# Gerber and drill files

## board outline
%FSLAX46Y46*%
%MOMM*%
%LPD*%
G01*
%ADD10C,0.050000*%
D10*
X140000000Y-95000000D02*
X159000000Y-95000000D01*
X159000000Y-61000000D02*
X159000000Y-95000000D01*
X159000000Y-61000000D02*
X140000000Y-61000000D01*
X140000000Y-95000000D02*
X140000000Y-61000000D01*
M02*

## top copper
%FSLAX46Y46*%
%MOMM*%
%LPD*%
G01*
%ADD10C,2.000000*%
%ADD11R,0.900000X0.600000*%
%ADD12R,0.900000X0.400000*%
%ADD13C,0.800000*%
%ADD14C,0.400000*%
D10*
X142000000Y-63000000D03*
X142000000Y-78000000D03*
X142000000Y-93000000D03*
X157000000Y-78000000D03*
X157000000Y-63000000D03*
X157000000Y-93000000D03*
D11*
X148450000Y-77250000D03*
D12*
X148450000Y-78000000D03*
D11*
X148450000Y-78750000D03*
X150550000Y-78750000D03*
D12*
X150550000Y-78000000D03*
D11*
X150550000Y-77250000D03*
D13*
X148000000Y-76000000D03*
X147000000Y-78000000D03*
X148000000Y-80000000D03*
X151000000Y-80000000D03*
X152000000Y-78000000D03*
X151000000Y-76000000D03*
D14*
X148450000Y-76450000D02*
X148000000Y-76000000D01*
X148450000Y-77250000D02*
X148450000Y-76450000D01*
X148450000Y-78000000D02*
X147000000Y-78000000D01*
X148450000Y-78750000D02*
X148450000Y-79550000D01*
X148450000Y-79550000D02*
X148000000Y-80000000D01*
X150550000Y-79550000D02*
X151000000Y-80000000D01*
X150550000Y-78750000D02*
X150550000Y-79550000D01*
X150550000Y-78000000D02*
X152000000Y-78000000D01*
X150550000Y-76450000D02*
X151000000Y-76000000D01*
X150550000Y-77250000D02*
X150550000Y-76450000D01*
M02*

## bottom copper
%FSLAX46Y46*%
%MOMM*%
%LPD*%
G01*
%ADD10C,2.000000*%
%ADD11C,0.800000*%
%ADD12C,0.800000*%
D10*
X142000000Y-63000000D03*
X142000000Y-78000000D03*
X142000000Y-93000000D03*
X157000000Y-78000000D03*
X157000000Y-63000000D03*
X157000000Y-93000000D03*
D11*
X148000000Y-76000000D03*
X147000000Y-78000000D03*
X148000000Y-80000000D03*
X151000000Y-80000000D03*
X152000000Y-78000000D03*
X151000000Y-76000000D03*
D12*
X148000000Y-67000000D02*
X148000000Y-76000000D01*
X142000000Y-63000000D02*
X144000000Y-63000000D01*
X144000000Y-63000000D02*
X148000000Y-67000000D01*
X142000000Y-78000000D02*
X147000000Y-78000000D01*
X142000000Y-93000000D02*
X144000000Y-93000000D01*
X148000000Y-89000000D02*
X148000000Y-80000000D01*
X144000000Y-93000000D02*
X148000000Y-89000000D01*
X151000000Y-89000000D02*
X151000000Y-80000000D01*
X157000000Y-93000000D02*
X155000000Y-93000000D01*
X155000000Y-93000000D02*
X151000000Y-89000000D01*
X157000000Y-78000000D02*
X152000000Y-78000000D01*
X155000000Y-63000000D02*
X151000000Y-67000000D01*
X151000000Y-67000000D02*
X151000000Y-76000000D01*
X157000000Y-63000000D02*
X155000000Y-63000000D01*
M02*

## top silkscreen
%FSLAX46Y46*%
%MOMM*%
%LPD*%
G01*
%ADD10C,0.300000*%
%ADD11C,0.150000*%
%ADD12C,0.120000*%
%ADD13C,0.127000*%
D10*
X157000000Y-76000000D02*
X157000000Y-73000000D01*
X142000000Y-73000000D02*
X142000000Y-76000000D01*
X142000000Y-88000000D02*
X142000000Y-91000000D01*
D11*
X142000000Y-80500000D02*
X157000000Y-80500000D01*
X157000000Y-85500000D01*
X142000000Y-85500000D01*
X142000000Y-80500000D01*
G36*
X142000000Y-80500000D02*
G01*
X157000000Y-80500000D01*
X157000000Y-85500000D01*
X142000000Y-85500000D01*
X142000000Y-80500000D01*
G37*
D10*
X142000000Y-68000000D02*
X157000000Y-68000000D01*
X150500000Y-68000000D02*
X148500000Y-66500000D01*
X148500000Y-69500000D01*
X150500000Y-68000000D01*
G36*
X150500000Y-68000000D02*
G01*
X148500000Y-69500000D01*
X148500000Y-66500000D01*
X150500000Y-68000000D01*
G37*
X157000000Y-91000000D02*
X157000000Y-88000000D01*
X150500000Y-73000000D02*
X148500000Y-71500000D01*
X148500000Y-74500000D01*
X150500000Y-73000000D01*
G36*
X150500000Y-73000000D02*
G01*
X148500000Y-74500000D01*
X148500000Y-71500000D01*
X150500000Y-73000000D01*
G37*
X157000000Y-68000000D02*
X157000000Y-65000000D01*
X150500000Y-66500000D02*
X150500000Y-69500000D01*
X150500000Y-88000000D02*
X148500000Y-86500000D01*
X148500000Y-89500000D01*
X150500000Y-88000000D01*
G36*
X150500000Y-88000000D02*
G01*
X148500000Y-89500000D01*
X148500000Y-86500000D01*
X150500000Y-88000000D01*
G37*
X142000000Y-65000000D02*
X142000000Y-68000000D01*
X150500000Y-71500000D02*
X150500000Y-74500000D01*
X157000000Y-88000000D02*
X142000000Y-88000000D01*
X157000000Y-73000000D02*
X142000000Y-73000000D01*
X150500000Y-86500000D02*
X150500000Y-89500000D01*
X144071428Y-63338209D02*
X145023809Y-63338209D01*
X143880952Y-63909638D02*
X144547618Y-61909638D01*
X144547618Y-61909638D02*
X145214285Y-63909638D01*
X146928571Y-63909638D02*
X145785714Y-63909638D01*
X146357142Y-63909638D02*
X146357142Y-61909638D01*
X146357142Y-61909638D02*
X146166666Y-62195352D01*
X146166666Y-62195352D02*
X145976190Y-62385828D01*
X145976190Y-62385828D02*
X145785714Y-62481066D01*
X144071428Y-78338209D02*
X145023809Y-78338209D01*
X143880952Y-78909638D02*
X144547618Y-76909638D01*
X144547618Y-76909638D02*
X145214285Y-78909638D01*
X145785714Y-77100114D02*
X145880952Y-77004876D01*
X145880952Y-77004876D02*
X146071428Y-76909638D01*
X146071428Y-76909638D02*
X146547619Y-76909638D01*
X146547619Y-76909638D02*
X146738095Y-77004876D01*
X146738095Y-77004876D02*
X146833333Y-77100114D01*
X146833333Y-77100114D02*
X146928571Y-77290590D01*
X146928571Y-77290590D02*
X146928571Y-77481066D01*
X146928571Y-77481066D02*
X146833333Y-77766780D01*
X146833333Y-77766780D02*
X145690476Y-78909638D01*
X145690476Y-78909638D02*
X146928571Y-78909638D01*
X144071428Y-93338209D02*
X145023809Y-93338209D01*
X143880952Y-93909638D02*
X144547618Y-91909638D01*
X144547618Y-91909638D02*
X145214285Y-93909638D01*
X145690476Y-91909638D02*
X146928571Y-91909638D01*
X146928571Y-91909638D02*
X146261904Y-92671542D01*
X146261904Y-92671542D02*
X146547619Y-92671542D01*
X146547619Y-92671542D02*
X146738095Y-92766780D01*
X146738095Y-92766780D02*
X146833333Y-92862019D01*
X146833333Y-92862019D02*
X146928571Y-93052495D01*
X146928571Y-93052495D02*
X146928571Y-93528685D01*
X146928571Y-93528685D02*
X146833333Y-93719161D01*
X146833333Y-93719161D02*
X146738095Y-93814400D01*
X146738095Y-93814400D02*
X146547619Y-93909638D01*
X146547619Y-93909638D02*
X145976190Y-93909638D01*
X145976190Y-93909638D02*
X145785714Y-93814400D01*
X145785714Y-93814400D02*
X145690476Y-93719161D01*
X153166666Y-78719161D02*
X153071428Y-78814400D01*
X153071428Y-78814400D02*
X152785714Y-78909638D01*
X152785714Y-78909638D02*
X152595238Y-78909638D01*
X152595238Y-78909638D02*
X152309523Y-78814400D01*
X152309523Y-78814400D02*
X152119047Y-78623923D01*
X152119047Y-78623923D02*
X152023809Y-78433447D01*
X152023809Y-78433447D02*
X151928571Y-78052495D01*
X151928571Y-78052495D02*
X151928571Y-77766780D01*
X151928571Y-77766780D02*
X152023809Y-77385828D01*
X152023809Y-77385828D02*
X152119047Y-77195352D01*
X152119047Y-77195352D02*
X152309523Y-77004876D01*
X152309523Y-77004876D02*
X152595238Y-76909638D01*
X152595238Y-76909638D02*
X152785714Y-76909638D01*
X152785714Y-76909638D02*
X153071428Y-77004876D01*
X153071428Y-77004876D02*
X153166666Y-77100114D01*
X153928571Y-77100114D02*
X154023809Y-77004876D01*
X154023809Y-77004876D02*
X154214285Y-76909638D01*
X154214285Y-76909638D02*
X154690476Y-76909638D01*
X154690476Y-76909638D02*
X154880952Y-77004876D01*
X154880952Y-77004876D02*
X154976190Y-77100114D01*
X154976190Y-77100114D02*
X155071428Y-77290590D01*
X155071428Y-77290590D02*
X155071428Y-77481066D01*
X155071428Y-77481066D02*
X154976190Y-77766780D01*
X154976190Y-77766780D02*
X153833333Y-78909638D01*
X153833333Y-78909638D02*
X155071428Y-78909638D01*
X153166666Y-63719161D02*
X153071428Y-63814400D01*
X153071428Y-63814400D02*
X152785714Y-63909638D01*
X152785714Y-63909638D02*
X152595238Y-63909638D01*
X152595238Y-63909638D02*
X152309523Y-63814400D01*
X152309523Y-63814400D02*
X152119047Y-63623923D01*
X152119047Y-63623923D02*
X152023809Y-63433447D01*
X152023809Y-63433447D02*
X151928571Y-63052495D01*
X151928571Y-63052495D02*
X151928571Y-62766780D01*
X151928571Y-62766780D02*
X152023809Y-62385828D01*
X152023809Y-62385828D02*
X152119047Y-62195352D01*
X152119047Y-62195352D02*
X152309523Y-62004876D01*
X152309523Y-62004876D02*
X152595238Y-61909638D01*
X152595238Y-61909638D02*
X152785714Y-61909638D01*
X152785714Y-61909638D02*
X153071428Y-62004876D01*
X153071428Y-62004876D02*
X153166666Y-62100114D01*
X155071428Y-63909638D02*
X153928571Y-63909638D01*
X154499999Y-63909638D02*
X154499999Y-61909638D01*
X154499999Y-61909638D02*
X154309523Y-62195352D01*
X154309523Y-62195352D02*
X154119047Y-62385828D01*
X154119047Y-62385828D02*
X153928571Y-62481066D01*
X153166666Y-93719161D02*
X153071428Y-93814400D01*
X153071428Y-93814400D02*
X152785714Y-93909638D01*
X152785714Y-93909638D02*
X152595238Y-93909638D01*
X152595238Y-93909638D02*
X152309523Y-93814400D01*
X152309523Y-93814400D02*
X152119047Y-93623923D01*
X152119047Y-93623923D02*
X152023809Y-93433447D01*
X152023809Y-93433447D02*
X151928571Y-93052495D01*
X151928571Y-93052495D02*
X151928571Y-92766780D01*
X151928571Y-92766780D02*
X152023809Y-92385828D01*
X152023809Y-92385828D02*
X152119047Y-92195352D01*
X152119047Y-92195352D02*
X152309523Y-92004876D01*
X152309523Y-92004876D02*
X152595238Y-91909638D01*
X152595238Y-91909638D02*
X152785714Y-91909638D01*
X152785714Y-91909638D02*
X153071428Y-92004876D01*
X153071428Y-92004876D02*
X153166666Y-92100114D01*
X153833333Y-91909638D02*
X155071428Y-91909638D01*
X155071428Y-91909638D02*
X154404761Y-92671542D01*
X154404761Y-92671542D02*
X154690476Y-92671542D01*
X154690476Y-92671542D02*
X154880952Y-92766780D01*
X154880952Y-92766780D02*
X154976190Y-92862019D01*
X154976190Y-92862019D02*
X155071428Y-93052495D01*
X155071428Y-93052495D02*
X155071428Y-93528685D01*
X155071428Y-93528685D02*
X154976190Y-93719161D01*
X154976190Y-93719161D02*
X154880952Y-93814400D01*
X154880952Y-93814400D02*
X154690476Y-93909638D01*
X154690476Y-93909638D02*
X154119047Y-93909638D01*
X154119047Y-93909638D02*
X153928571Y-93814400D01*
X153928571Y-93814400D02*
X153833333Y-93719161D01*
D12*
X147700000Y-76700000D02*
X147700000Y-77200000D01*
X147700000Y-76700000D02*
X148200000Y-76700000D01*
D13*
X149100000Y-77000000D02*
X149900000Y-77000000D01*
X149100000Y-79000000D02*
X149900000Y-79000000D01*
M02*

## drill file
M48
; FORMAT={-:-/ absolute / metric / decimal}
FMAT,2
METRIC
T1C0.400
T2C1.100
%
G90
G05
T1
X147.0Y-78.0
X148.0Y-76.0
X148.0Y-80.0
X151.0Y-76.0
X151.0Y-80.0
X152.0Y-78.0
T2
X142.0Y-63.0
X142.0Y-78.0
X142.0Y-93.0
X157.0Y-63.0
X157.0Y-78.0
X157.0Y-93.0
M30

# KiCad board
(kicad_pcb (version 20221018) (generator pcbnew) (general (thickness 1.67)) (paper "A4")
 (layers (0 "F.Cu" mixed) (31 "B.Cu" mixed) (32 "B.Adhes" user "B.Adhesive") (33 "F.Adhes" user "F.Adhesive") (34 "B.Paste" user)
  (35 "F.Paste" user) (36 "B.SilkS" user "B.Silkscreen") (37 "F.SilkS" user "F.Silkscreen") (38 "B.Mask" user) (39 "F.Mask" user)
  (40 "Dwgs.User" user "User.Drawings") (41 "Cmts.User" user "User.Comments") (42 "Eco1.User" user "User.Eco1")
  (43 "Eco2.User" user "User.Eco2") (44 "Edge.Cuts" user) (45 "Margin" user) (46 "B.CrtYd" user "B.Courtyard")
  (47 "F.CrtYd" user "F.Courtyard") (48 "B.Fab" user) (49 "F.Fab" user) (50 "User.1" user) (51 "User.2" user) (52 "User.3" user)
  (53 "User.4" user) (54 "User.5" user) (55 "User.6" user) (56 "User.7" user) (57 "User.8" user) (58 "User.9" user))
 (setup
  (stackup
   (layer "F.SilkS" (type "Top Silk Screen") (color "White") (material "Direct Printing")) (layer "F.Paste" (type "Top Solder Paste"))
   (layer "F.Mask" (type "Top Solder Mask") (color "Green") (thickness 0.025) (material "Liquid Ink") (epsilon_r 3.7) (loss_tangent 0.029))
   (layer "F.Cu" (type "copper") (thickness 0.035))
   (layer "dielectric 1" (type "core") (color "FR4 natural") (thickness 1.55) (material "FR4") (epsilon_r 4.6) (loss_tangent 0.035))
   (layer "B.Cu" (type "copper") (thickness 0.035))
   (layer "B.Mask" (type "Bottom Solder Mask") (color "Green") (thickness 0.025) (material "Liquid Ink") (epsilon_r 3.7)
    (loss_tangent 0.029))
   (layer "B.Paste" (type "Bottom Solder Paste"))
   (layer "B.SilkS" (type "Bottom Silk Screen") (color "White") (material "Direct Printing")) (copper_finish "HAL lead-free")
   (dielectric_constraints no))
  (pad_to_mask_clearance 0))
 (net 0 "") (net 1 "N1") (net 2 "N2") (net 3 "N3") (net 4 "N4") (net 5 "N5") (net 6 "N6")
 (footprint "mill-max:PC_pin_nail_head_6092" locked (layer "F.Cu") (at 142 63)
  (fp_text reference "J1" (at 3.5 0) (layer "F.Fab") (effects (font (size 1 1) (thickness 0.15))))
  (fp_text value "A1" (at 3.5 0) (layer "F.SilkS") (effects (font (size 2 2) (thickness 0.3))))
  (pad "1" thru_hole circle locked (at 0 0) (size 2 2) (drill 1.1) (layers "*.Cu" "*.Mask") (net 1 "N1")))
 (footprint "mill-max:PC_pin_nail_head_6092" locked (layer "F.Cu") (at 142 78)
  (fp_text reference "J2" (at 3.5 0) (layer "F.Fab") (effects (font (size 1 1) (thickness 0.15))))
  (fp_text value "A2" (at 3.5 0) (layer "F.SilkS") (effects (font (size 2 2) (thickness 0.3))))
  (pad "1" thru_hole circle locked (at 0 0) (size 2 2) (drill 1.1) (layers "*.Cu" "*.Mask") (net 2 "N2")))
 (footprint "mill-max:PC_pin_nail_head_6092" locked (layer "F.Cu") (at 142 93)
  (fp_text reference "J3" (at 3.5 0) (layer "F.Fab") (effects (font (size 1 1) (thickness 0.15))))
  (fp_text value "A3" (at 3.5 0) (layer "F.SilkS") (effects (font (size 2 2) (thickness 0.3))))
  (pad "1" thru_hole circle locked (at 0 0) (size 2 2) (drill 1.1) (layers "*.Cu" "*.Mask") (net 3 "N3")))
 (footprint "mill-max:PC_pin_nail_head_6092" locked (layer "F.Cu") (at 157 78)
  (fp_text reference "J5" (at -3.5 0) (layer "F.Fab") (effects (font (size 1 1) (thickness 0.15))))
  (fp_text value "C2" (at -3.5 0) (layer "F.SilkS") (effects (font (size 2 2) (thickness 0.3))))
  (pad "1" thru_hole circle locked (at 0 0) (size 2 2) (drill 1.1) (layers "*.Cu" "*.Mask") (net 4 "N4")))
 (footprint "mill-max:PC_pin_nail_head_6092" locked (layer "F.Cu") (at 157 63)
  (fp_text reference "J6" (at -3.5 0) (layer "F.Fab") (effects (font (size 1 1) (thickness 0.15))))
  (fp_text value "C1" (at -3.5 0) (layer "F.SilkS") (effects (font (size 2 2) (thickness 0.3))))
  (pad "1" thru_hole circle locked (at 0 0) (size 2 2) (drill 1.1) (layers "*.Cu" "*.Mask") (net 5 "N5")))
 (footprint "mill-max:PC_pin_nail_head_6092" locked (layer "F.Cu") (at 157 93)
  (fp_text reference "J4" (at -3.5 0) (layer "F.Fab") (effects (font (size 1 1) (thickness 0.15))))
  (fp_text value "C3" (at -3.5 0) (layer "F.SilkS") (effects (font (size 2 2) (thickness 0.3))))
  (pad "1" thru_hole circle locked (at 0 0) (size 2 2) (drill 1.1) (layers "*.Cu" "*.Mask") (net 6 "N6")))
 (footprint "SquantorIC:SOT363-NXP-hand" (layer "F.Cu") (at 149.5 78)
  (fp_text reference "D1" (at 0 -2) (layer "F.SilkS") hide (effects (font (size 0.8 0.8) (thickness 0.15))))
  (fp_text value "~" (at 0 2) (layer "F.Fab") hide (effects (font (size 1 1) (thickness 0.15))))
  (fp_line (start -1.8 -1.3) (end -1.8 -0.8) (stroke (width 0.12) (type solid)) (layer "F.SilkS"))
  (fp_line (start -1.8 -1.3) (end -1.3 -1.3) (stroke (width 0.12) (type solid)) (layer "F.SilkS"))
  (fp_line (start -0.4 -1) (end 0.4 -1) (stroke (width 0.127) (type solid)) (layer "F.SilkS"))
  (fp_line (start -0.4 1) (end 0.4 1) (stroke (width 0.127) (type solid)) (layer "F.SilkS"))
  (pad "1" smd rect (at -1.05 -0.75 270) (size 0.6 0.9) (layers "F.Cu" "F.Paste" "F.Mask") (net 1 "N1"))
  (pad "2" smd rect (at -1.05 0 270) (size 0.4 0.9) (layers "F.Cu" "F.Paste" "F.Mask") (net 2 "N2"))
  (pad "3" smd rect (at -1.05 0.75 270) (size 0.6 0.9) (layers "F.Cu" "F.Paste" "F.Mask") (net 3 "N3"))
  (pad "4" smd rect (at 1.05 0.75 270) (size 0.6 0.9) (layers "F.Cu" "F.Paste" "F.Mask") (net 6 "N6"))
  (pad "5" smd rect (at 1.05 0 270) (size 0.4 0.9) (layers "F.Cu" "F.Paste" "F.Mask") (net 4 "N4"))
  (pad "6" smd rect (at 1.05 -0.75 270) (size 0.6 0.9) (layers "F.Cu" "F.Paste" "F.Mask") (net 5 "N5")))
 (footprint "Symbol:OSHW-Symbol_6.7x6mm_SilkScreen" (layer "B.Cu") (at 149.5 77 180)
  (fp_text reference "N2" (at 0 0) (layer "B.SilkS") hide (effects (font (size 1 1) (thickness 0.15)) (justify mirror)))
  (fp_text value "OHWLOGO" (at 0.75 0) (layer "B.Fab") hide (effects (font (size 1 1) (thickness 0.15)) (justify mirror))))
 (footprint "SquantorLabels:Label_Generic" (layer "B.Cu") (at 149.5 80.5)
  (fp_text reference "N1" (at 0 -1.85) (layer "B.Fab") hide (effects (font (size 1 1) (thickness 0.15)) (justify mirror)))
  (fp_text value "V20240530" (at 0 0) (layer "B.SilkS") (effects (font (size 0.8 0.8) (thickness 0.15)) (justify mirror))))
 (gr_line (start 157 76) (end 157 73) (stroke (width 0.3) (type default)) (layer "F.SilkS"))
 (gr_line (start 142 73) (end 142 76) (stroke (width 0.3) (type default)) (layer "F.SilkS"))
 (gr_line (start 142 88) (end 142 91) (stroke (width 0.3) (type default)) (layer "F.SilkS"))
 (gr_rect (start 142 80.5) (end 157 85.5) (stroke (width 0.15) (type solid)) (fill solid) (layer "F.SilkS"))
 (gr_line (start 142 68) (end 157 68) (stroke (width 0.3) (type default)) (layer "F.SilkS"))
 (gr_poly (pts (xy 150.5 68) (xy 148.5 66.5) (xy 148.5 69.5)) (stroke (width 0.3) (type solid)) (fill solid) (layer "F.SilkS"))
 (gr_line (start 157 91) (end 157 88) (stroke (width 0.3) (type default)) (layer "F.SilkS"))
 (gr_poly (pts (xy 150.5 73) (xy 148.5 71.5) (xy 148.5 74.5)) (stroke (width 0.3) (type solid)) (fill solid) (layer "F.SilkS"))
 (gr_line (start 157 68) (end 157 65) (stroke (width 0.3) (type default)) (layer "F.SilkS"))
 (gr_line (start 150.5 66.5) (end 150.5 69.5) (stroke (width 0.3) (type default)) (layer "F.SilkS"))
 (gr_poly (pts (xy 150.5 88) (xy 148.5 86.5) (xy 148.5 89.5)) (stroke (width 0.3) (type solid)) (fill solid) (layer "F.SilkS"))
 (gr_line (start 142 65) (end 142 68) (stroke (width 0.3) (type default)) (layer "F.SilkS"))
 (gr_line (start 150.5 71.5) (end 150.5 74.5) (stroke (width 0.3) (type default)) (layer "F.SilkS"))
 (gr_line (start 157 88) (end 142 88) (stroke (width 0.3) (type default)) (layer "F.SilkS"))
 (gr_line (start 157 73) (end 142 73) (stroke (width 0.3) (type default)) (layer "F.SilkS"))
 (gr_line (start 150.5 86.5) (end 150.5 89.5) (stroke (width 0.3) (type default)) (layer "F.SilkS"))
 (gr_line (start 140 95) (end 159 95) (stroke (width 0.05) (type solid)) (layer "Edge.Cuts"))
 (gr_line (start 159 61) (end 159 95) (stroke (width 0.05) (type solid)) (layer "Edge.Cuts"))
 (gr_line (start 159 61) (end 140 61) (stroke (width 0.05) (type solid)) (layer "Edge.Cuts"))
 (gr_line (start 140 95) (end 140 61) (stroke (width 0.05) (type solid)) (layer "Edge.Cuts"))
 (segment (start 148.45 76.45) (end 148 76) (width 0.4) (layer "F.Cu") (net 1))
 (segment (start 148.45 77.25) (end 148.45 76.45) (width 0.4) (layer "F.Cu") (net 1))
 (via (at 148 76) (size 0.8) (drill 0.4) (layers "F.Cu" "B.Cu") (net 1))
 (segment (start 148 67) (end 148 76) (width 0.8) (layer "B.Cu") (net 1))
 (segment (start 142 63) (end 144 63) (width 0.8) (layer "B.Cu") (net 1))
 (segment (start 144 63) (end 148 67) (width 0.8) (layer "B.Cu") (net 1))
 (segment (start 148.45 78) (end 147 78) (width 0.4) (layer "F.Cu") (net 2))
 (via (at 147 78) (size 0.8) (drill 0.4) (layers "F.Cu" "B.Cu") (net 2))
 (segment (start 142 78) (end 147 78) (width 0.8) (layer "B.Cu") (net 2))
 (segment (start 148.45 78.75) (end 148.45 79.55) (width 0.4) (layer "F.Cu") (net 3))
 (segment (start 148.45 79.55) (end 148 80) (width 0.4) (layer "F.Cu") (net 3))
 (via (at 148 80) (size 0.8) (drill 0.4) (layers "F.Cu" "B.Cu") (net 3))
 (segment (start 142 93) (end 144 93) (width 0.8) (layer "B.Cu") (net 3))
 (segment (start 148 89) (end 148 80) (width 0.8) (layer "B.Cu") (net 3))
 (segment (start 144 93) (end 148 89) (width 0.8) (layer "B.Cu") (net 3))
 (segment (start 150.55 79.55) (end 151 80) (width 0.4) (layer "F.Cu") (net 6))
 (segment (start 150.55 78.75) (end 150.55 79.55) (width 0.4) (layer "F.Cu") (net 6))
 (via (at 151 80) (size 0.8) (drill 0.4) (layers "F.Cu" "B.Cu") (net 6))
 (segment (start 151 89) (end 151 80) (width 0.8) (layer "B.Cu") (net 6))
 (segment (start 157 93) (end 155 93) (width 0.8) (layer "B.Cu") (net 6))
 (segment (start 155 93) (end 151 89) (width 0.8) (layer "B.Cu") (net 6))
 (segment (start 150.55 78) (end 152 78) (width 0.4) (layer "F.Cu") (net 4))
 (via (at 152 78) (size 0.8) (drill 0.4) (layers "F.Cu" "B.Cu") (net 4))
 (segment (start 157 78) (end 152 78) (width 0.8) (layer "B.Cu") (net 4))
 (segment (start 150.55 76.45) (end 151 76) (width 0.4) (layer "F.Cu") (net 5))
 (segment (start 150.55 77.25) (end 150.55 76.45) (width 0.4) (layer "F.Cu") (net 5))
 (via (at 151 76) (size 0.8) (drill 0.4) (layers "F.Cu" "B.Cu") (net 5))
 (segment (start 155 63) (end 151 67) (width 0.8) (layer "B.Cu") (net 5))
 (segment (start 151 67) (end 151 76) (width 0.8) (layer "B.Cu") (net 5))
 (segment (start 157 63) (end 155 63) (width 0.8) (layer "B.Cu") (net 5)))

